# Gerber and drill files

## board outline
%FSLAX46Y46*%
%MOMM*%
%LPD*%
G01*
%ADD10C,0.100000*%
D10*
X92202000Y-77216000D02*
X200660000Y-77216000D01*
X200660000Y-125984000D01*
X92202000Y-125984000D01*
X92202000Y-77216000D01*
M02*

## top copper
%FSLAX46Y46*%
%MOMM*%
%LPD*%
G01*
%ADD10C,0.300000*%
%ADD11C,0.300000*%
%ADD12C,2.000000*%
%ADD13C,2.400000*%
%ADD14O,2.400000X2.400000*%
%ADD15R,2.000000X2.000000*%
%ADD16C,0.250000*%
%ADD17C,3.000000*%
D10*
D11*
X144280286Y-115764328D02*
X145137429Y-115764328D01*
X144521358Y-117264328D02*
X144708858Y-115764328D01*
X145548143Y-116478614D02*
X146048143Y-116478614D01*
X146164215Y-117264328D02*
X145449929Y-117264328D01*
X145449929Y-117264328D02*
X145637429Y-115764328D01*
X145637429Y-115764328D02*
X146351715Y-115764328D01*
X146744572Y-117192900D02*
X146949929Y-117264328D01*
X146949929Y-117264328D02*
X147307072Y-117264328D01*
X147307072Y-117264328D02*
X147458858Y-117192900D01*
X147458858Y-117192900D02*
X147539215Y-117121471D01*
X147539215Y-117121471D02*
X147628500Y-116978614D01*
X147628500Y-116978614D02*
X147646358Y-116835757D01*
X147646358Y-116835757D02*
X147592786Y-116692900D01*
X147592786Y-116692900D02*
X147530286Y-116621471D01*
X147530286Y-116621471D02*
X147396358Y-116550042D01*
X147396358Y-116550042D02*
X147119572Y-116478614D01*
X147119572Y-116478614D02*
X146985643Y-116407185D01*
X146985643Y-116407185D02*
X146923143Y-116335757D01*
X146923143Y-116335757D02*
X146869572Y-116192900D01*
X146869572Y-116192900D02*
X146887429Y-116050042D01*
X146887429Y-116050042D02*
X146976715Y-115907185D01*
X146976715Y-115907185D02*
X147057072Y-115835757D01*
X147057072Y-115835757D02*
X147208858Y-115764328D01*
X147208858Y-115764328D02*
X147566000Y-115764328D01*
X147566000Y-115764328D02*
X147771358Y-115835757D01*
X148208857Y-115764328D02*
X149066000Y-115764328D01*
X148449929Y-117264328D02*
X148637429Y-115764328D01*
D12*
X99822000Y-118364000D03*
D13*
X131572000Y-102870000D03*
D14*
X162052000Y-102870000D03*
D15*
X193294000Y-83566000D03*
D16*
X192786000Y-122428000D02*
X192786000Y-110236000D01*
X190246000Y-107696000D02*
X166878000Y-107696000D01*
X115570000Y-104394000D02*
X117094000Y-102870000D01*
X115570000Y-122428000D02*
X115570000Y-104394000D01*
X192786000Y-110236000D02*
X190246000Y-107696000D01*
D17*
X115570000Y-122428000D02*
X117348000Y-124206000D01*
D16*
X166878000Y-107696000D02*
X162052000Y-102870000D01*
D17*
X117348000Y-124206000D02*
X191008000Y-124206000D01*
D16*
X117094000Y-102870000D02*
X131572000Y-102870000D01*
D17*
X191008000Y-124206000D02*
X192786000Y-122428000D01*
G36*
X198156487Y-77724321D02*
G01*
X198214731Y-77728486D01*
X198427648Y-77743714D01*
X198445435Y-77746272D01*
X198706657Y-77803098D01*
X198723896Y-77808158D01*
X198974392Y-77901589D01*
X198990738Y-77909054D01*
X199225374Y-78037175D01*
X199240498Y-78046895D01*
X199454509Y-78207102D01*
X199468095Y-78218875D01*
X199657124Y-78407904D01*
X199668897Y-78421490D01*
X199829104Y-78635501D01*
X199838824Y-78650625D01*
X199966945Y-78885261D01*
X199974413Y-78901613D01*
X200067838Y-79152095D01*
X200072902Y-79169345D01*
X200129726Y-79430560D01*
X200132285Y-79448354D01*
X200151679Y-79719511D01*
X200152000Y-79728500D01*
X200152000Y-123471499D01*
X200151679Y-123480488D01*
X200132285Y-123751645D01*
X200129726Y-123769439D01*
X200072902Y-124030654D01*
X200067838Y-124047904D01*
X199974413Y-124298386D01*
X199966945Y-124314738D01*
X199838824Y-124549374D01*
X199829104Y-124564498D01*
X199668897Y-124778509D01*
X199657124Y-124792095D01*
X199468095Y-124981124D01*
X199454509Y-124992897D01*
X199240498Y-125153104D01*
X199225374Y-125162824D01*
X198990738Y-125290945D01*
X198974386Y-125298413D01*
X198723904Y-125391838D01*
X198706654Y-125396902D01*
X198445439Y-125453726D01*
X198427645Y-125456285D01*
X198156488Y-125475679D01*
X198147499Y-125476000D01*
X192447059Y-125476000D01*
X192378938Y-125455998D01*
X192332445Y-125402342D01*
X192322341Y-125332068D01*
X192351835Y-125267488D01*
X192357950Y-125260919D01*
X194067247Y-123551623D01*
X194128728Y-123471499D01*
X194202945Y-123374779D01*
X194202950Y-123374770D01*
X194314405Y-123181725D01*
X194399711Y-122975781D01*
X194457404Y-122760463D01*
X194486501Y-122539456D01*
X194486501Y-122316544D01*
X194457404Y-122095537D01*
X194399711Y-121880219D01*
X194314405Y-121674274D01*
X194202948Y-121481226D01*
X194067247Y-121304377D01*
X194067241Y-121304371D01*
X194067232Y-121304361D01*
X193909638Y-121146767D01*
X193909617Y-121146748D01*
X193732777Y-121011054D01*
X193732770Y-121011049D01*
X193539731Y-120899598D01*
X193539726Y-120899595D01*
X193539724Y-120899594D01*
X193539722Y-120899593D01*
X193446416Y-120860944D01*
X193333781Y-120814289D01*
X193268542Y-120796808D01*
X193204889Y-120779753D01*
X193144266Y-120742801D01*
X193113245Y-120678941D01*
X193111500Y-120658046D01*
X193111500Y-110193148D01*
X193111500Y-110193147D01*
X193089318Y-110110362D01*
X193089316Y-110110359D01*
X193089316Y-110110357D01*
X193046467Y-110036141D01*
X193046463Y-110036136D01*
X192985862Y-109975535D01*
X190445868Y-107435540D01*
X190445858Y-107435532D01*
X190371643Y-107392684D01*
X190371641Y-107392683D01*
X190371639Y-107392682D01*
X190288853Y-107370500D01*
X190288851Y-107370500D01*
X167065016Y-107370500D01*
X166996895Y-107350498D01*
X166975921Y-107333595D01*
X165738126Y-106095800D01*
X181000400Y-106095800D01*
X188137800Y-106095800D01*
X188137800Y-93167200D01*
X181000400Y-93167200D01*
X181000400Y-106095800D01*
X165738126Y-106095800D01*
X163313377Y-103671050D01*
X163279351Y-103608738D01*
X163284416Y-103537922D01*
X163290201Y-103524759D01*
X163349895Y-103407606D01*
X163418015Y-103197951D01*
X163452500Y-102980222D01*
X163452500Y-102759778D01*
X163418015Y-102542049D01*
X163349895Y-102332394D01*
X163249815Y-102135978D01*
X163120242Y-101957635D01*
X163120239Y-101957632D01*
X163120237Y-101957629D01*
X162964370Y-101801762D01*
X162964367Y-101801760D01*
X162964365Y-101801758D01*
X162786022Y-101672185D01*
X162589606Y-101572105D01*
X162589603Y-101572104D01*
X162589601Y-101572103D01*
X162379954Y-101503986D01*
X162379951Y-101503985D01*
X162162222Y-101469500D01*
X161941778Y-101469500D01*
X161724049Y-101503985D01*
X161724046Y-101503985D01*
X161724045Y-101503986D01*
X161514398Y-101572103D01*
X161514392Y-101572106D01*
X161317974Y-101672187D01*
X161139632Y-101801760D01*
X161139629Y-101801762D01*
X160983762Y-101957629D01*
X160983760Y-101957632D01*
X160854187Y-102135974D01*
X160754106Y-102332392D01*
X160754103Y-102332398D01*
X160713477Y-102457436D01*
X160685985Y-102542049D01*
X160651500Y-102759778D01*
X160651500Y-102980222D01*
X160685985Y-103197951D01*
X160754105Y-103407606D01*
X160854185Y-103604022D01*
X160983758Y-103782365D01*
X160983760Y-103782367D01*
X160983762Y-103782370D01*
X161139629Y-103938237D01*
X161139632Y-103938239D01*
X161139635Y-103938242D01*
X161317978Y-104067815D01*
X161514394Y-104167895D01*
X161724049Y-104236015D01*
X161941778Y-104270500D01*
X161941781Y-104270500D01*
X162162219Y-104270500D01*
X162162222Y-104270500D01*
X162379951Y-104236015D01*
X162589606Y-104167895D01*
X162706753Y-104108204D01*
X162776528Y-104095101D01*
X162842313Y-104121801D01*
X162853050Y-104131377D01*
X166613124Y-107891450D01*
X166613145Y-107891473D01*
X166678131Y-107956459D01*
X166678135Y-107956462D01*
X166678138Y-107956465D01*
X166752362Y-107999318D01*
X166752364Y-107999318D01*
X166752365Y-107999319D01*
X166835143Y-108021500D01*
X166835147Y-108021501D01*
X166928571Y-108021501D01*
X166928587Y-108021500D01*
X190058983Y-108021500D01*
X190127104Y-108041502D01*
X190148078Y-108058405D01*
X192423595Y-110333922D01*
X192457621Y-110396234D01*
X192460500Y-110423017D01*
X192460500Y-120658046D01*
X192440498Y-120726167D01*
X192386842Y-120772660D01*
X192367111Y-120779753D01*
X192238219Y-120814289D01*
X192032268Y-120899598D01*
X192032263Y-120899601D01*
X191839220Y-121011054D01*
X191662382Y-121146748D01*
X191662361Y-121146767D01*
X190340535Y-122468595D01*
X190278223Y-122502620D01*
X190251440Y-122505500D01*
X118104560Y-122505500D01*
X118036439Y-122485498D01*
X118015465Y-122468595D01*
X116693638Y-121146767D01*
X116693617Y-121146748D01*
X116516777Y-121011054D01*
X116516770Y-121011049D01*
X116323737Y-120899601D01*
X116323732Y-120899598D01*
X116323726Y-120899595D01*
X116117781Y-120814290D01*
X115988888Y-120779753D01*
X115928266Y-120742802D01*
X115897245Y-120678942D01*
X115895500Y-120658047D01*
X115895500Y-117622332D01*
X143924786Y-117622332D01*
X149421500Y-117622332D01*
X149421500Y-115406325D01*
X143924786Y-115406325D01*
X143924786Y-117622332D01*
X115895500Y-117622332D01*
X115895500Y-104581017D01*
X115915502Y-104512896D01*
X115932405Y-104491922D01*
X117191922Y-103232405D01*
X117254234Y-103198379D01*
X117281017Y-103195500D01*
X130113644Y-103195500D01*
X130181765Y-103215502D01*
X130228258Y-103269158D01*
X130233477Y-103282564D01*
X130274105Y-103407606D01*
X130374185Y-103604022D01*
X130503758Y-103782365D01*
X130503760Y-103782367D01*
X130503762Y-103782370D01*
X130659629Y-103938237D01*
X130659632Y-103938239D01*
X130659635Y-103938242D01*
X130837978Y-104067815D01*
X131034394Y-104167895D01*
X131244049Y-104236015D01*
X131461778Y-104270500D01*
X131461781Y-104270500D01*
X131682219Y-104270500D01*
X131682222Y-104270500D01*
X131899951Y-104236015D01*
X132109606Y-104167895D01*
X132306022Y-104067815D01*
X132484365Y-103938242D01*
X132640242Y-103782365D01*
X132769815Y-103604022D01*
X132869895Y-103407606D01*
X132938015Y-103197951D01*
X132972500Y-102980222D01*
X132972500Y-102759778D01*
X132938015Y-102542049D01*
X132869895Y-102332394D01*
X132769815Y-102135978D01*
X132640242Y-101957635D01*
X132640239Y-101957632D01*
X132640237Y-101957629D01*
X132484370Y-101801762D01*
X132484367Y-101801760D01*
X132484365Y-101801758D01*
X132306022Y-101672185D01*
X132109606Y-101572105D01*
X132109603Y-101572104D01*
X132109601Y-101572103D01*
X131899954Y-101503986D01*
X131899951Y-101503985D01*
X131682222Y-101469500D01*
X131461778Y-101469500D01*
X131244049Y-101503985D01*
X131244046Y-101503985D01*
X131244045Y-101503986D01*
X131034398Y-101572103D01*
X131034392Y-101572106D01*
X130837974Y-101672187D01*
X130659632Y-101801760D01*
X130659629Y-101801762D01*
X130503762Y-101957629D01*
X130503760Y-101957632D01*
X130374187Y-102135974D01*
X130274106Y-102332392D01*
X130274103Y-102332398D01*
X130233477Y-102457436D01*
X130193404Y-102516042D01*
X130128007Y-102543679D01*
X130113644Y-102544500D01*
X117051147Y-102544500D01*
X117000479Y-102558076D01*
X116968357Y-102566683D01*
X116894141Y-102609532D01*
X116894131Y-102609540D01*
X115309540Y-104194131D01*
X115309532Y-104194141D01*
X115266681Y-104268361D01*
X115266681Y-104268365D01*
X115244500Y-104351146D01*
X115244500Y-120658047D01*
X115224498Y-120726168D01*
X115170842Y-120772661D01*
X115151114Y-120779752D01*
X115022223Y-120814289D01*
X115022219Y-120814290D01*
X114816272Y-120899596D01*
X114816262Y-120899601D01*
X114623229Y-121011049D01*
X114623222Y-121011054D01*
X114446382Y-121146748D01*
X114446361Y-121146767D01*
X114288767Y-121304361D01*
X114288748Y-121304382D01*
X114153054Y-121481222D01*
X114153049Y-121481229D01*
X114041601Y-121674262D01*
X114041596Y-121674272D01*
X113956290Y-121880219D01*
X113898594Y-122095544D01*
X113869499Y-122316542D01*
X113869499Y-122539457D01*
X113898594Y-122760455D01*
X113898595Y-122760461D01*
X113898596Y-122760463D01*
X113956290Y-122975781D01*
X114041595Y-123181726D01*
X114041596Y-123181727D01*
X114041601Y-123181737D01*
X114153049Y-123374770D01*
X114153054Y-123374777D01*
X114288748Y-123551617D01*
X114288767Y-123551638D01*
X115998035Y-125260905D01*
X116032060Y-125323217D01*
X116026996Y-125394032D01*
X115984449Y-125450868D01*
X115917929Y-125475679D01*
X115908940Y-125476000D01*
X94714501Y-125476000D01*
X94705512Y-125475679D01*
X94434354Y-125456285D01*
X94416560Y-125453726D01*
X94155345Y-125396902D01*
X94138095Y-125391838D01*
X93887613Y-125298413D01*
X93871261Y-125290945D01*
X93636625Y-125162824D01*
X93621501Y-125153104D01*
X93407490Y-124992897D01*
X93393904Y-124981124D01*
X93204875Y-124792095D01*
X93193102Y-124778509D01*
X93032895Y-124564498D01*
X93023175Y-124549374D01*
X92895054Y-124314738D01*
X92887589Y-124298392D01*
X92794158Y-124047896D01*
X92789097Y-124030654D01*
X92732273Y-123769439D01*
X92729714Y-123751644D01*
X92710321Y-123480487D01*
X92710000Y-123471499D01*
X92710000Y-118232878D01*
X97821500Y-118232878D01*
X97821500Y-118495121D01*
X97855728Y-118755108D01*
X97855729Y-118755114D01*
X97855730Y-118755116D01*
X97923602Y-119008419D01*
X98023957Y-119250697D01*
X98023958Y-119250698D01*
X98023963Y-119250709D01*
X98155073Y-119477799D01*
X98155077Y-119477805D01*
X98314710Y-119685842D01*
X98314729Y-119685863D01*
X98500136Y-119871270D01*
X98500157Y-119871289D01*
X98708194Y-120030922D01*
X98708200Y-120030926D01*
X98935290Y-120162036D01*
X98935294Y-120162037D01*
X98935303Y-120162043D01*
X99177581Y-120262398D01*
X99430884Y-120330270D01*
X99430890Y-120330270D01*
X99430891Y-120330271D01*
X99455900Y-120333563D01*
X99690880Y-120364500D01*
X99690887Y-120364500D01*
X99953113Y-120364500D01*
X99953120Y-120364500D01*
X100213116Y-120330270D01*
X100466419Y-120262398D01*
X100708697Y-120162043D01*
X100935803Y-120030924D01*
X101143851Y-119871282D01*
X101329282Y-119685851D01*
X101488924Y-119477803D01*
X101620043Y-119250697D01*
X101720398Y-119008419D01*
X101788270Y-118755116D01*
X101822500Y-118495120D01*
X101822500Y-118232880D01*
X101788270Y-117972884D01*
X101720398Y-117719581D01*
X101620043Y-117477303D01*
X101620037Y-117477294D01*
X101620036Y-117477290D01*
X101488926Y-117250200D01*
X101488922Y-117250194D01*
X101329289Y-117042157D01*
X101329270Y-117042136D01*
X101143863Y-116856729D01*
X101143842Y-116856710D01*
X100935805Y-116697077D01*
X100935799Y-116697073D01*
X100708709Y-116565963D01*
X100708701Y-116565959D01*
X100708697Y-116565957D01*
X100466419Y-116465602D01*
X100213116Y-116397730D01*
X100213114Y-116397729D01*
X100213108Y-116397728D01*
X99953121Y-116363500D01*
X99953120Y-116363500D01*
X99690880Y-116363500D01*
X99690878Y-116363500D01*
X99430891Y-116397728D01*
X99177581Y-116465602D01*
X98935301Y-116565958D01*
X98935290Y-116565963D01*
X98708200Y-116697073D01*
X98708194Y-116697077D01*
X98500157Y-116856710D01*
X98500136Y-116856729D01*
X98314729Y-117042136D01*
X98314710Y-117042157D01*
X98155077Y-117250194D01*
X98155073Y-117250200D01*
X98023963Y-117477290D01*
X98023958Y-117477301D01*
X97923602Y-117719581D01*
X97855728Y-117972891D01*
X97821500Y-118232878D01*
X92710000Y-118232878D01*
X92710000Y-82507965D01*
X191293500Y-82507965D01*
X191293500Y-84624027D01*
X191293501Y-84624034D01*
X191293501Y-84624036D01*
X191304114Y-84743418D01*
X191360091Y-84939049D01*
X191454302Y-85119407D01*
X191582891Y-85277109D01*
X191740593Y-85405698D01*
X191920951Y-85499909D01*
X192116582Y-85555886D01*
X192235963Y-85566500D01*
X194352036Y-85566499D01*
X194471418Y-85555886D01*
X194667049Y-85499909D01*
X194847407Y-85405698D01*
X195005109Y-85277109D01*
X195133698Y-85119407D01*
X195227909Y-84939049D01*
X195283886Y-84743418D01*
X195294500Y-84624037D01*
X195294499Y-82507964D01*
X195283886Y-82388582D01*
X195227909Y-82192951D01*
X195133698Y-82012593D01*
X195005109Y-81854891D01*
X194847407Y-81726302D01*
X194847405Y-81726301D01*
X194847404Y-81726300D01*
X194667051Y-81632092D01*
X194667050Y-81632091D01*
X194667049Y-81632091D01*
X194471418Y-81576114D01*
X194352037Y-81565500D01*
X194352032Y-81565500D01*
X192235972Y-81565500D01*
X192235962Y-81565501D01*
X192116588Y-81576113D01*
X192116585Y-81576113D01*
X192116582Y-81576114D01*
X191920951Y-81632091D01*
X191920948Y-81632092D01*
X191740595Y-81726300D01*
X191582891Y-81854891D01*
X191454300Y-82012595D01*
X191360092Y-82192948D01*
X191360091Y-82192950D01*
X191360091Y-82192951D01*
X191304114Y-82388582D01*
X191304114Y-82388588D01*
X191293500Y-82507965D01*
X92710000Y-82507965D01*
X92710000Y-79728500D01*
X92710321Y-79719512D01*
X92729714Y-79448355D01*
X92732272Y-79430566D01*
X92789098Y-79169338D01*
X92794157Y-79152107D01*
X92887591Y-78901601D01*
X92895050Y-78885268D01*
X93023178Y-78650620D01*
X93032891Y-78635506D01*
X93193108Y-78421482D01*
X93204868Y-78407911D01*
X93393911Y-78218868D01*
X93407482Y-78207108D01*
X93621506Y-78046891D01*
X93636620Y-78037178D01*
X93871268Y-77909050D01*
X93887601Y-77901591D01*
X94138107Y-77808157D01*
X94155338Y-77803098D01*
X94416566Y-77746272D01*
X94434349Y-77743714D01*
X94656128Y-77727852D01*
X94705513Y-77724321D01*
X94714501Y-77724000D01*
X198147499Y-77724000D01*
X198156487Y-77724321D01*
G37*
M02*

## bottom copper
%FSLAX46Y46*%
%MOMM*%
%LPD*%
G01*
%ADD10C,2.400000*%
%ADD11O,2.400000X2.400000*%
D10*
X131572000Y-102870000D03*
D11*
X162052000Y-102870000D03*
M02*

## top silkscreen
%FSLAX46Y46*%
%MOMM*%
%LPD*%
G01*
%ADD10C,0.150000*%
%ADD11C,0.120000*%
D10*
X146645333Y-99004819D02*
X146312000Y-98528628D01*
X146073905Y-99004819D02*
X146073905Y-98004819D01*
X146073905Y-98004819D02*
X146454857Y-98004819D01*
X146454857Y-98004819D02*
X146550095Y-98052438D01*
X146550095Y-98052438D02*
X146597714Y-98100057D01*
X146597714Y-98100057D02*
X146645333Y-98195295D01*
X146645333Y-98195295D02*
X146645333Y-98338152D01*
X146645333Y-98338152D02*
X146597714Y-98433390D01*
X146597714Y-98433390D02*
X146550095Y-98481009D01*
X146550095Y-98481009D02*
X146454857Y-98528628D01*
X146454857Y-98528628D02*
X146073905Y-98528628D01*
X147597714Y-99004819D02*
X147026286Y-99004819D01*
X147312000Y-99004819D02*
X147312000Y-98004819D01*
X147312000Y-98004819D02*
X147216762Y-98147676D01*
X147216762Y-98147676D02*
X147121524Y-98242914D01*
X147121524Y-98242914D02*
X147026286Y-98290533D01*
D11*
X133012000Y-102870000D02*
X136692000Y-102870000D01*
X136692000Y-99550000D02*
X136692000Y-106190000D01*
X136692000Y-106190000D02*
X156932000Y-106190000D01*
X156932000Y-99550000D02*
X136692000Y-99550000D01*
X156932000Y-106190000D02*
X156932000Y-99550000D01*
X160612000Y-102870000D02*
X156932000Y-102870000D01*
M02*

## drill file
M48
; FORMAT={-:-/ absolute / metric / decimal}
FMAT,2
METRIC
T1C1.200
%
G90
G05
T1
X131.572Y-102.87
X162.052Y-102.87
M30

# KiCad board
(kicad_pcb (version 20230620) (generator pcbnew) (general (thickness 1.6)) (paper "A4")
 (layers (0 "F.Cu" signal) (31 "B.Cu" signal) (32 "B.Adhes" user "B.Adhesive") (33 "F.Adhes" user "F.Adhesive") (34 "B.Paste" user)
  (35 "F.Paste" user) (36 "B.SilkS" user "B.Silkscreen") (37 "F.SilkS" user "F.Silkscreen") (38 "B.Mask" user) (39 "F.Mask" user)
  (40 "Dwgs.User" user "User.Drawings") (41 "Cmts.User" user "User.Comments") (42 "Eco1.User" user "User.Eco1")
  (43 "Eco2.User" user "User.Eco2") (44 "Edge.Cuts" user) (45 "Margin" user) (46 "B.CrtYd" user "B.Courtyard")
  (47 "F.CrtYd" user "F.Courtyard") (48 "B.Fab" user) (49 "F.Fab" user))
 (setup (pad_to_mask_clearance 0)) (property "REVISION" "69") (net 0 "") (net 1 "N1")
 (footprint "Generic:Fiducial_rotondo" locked (layer "F.Cu") (at 99.822 118.364)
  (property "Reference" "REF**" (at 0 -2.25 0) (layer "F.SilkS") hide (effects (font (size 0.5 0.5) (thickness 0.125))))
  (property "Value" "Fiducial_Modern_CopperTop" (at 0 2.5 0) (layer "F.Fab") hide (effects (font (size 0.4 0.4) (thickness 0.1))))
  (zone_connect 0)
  (pad "~" smd circle locked (at 0 0) (size 2 2) (layers "F.Cu" "F.Mask") (solder_mask_margin 1) (clearance 1) (zone_connect 0)))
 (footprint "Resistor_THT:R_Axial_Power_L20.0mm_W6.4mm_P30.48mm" (layer "F.Cu") (at 131.572 102.87)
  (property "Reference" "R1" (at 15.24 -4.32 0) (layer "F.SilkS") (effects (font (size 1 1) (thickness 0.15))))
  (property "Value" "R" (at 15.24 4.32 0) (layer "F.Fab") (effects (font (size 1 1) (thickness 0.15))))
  (fp_line (start 1.44 0) (end 5.12 0) (stroke (width 0.12) (type solid)) (layer "F.SilkS"))
  (fp_line (start 5.12 -3.32) (end 5.12 3.32) (stroke (width 0.12) (type solid)) (layer "F.SilkS"))
  (fp_line (start 5.12 3.32) (end 25.36 3.32) (stroke (width 0.12) (type solid)) (layer "F.SilkS"))
  (fp_line (start 25.36 -3.32) (end 5.12 -3.32) (stroke (width 0.12) (type solid)) (layer "F.SilkS"))
  (fp_line (start 25.36 3.32) (end 25.36 -3.32) (stroke (width 0.12) (type solid)) (layer "F.SilkS"))
  (fp_line (start 29.04 0) (end 25.36 0) (stroke (width 0.12) (type solid)) (layer "F.SilkS"))
  (pad "1" thru_hole circle (at 0 0) (size 2.4 2.4) (drill 1.2) (layers "*.Cu" "*.Mask") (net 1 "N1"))
  (pad "2" thru_hole oval (at 30.48 0) (size 2.4 2.4) (drill 1.2) (layers "*.Cu" "*.Mask") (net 1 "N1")))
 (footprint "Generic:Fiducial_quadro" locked (layer "F.Cu") (at 193.294 83.566)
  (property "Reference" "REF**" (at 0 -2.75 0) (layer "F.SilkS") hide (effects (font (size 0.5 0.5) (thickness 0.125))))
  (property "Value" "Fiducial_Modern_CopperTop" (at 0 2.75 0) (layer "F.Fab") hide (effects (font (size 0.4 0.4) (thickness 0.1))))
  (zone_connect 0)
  (pad "~" smd rect locked (at 0 0) (size 2 2) (layers "F.Cu" "F.Mask") (solder_mask_margin 1) (clearance 1) (zone_connect 0)))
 (gr_rect (start 92.202 77.216) (end 200.66 125.984) (stroke (width 0.1) (type solid)) (fill none) (layer "Edge.Cuts"))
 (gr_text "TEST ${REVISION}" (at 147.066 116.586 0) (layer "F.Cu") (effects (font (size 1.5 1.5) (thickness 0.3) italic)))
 (segment (start 192.786 122.428) (end 192.786 110.236) (width 0.25) (layer "F.Cu") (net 1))
 (segment (start 190.246 107.696) (end 166.878 107.696) (width 0.25) (layer "F.Cu") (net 1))
 (segment (start 115.57 104.394) (end 117.094 102.87) (width 0.25) (layer "F.Cu") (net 1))
 (segment (start 115.57 122.428) (end 115.57 104.394) (width 0.25) (layer "F.Cu") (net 1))
 (segment (start 192.786 110.236) (end 190.246 107.696) (width 0.25) (layer "F.Cu") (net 1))
 (segment (start 115.57 122.428) (end 117.348 124.206) (width 3) (layer "F.Cu") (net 1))
 (segment (start 166.878 107.696) (end 162.052 102.87) (width 0.25) (layer "F.Cu") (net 1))
 (segment (start 117.348 124.206) (end 191.008 124.206) (width 3) (layer "F.Cu") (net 1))
 (segment (start 117.094 102.87) (end 131.572 102.87) (width 0.25) (layer "F.Cu") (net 1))
 (segment (start 191.008 124.206) (end 192.786 122.428) (width 3) (layer "F.Cu") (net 1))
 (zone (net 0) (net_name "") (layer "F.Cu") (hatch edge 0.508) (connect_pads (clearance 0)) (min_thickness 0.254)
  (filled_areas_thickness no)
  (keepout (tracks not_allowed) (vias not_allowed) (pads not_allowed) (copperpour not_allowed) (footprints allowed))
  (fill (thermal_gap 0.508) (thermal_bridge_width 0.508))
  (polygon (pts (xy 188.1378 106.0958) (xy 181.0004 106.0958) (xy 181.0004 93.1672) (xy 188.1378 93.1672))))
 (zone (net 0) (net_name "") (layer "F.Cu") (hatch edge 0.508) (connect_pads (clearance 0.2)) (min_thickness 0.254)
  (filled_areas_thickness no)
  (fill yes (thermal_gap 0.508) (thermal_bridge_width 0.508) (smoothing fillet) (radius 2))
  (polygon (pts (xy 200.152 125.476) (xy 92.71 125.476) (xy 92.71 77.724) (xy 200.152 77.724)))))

